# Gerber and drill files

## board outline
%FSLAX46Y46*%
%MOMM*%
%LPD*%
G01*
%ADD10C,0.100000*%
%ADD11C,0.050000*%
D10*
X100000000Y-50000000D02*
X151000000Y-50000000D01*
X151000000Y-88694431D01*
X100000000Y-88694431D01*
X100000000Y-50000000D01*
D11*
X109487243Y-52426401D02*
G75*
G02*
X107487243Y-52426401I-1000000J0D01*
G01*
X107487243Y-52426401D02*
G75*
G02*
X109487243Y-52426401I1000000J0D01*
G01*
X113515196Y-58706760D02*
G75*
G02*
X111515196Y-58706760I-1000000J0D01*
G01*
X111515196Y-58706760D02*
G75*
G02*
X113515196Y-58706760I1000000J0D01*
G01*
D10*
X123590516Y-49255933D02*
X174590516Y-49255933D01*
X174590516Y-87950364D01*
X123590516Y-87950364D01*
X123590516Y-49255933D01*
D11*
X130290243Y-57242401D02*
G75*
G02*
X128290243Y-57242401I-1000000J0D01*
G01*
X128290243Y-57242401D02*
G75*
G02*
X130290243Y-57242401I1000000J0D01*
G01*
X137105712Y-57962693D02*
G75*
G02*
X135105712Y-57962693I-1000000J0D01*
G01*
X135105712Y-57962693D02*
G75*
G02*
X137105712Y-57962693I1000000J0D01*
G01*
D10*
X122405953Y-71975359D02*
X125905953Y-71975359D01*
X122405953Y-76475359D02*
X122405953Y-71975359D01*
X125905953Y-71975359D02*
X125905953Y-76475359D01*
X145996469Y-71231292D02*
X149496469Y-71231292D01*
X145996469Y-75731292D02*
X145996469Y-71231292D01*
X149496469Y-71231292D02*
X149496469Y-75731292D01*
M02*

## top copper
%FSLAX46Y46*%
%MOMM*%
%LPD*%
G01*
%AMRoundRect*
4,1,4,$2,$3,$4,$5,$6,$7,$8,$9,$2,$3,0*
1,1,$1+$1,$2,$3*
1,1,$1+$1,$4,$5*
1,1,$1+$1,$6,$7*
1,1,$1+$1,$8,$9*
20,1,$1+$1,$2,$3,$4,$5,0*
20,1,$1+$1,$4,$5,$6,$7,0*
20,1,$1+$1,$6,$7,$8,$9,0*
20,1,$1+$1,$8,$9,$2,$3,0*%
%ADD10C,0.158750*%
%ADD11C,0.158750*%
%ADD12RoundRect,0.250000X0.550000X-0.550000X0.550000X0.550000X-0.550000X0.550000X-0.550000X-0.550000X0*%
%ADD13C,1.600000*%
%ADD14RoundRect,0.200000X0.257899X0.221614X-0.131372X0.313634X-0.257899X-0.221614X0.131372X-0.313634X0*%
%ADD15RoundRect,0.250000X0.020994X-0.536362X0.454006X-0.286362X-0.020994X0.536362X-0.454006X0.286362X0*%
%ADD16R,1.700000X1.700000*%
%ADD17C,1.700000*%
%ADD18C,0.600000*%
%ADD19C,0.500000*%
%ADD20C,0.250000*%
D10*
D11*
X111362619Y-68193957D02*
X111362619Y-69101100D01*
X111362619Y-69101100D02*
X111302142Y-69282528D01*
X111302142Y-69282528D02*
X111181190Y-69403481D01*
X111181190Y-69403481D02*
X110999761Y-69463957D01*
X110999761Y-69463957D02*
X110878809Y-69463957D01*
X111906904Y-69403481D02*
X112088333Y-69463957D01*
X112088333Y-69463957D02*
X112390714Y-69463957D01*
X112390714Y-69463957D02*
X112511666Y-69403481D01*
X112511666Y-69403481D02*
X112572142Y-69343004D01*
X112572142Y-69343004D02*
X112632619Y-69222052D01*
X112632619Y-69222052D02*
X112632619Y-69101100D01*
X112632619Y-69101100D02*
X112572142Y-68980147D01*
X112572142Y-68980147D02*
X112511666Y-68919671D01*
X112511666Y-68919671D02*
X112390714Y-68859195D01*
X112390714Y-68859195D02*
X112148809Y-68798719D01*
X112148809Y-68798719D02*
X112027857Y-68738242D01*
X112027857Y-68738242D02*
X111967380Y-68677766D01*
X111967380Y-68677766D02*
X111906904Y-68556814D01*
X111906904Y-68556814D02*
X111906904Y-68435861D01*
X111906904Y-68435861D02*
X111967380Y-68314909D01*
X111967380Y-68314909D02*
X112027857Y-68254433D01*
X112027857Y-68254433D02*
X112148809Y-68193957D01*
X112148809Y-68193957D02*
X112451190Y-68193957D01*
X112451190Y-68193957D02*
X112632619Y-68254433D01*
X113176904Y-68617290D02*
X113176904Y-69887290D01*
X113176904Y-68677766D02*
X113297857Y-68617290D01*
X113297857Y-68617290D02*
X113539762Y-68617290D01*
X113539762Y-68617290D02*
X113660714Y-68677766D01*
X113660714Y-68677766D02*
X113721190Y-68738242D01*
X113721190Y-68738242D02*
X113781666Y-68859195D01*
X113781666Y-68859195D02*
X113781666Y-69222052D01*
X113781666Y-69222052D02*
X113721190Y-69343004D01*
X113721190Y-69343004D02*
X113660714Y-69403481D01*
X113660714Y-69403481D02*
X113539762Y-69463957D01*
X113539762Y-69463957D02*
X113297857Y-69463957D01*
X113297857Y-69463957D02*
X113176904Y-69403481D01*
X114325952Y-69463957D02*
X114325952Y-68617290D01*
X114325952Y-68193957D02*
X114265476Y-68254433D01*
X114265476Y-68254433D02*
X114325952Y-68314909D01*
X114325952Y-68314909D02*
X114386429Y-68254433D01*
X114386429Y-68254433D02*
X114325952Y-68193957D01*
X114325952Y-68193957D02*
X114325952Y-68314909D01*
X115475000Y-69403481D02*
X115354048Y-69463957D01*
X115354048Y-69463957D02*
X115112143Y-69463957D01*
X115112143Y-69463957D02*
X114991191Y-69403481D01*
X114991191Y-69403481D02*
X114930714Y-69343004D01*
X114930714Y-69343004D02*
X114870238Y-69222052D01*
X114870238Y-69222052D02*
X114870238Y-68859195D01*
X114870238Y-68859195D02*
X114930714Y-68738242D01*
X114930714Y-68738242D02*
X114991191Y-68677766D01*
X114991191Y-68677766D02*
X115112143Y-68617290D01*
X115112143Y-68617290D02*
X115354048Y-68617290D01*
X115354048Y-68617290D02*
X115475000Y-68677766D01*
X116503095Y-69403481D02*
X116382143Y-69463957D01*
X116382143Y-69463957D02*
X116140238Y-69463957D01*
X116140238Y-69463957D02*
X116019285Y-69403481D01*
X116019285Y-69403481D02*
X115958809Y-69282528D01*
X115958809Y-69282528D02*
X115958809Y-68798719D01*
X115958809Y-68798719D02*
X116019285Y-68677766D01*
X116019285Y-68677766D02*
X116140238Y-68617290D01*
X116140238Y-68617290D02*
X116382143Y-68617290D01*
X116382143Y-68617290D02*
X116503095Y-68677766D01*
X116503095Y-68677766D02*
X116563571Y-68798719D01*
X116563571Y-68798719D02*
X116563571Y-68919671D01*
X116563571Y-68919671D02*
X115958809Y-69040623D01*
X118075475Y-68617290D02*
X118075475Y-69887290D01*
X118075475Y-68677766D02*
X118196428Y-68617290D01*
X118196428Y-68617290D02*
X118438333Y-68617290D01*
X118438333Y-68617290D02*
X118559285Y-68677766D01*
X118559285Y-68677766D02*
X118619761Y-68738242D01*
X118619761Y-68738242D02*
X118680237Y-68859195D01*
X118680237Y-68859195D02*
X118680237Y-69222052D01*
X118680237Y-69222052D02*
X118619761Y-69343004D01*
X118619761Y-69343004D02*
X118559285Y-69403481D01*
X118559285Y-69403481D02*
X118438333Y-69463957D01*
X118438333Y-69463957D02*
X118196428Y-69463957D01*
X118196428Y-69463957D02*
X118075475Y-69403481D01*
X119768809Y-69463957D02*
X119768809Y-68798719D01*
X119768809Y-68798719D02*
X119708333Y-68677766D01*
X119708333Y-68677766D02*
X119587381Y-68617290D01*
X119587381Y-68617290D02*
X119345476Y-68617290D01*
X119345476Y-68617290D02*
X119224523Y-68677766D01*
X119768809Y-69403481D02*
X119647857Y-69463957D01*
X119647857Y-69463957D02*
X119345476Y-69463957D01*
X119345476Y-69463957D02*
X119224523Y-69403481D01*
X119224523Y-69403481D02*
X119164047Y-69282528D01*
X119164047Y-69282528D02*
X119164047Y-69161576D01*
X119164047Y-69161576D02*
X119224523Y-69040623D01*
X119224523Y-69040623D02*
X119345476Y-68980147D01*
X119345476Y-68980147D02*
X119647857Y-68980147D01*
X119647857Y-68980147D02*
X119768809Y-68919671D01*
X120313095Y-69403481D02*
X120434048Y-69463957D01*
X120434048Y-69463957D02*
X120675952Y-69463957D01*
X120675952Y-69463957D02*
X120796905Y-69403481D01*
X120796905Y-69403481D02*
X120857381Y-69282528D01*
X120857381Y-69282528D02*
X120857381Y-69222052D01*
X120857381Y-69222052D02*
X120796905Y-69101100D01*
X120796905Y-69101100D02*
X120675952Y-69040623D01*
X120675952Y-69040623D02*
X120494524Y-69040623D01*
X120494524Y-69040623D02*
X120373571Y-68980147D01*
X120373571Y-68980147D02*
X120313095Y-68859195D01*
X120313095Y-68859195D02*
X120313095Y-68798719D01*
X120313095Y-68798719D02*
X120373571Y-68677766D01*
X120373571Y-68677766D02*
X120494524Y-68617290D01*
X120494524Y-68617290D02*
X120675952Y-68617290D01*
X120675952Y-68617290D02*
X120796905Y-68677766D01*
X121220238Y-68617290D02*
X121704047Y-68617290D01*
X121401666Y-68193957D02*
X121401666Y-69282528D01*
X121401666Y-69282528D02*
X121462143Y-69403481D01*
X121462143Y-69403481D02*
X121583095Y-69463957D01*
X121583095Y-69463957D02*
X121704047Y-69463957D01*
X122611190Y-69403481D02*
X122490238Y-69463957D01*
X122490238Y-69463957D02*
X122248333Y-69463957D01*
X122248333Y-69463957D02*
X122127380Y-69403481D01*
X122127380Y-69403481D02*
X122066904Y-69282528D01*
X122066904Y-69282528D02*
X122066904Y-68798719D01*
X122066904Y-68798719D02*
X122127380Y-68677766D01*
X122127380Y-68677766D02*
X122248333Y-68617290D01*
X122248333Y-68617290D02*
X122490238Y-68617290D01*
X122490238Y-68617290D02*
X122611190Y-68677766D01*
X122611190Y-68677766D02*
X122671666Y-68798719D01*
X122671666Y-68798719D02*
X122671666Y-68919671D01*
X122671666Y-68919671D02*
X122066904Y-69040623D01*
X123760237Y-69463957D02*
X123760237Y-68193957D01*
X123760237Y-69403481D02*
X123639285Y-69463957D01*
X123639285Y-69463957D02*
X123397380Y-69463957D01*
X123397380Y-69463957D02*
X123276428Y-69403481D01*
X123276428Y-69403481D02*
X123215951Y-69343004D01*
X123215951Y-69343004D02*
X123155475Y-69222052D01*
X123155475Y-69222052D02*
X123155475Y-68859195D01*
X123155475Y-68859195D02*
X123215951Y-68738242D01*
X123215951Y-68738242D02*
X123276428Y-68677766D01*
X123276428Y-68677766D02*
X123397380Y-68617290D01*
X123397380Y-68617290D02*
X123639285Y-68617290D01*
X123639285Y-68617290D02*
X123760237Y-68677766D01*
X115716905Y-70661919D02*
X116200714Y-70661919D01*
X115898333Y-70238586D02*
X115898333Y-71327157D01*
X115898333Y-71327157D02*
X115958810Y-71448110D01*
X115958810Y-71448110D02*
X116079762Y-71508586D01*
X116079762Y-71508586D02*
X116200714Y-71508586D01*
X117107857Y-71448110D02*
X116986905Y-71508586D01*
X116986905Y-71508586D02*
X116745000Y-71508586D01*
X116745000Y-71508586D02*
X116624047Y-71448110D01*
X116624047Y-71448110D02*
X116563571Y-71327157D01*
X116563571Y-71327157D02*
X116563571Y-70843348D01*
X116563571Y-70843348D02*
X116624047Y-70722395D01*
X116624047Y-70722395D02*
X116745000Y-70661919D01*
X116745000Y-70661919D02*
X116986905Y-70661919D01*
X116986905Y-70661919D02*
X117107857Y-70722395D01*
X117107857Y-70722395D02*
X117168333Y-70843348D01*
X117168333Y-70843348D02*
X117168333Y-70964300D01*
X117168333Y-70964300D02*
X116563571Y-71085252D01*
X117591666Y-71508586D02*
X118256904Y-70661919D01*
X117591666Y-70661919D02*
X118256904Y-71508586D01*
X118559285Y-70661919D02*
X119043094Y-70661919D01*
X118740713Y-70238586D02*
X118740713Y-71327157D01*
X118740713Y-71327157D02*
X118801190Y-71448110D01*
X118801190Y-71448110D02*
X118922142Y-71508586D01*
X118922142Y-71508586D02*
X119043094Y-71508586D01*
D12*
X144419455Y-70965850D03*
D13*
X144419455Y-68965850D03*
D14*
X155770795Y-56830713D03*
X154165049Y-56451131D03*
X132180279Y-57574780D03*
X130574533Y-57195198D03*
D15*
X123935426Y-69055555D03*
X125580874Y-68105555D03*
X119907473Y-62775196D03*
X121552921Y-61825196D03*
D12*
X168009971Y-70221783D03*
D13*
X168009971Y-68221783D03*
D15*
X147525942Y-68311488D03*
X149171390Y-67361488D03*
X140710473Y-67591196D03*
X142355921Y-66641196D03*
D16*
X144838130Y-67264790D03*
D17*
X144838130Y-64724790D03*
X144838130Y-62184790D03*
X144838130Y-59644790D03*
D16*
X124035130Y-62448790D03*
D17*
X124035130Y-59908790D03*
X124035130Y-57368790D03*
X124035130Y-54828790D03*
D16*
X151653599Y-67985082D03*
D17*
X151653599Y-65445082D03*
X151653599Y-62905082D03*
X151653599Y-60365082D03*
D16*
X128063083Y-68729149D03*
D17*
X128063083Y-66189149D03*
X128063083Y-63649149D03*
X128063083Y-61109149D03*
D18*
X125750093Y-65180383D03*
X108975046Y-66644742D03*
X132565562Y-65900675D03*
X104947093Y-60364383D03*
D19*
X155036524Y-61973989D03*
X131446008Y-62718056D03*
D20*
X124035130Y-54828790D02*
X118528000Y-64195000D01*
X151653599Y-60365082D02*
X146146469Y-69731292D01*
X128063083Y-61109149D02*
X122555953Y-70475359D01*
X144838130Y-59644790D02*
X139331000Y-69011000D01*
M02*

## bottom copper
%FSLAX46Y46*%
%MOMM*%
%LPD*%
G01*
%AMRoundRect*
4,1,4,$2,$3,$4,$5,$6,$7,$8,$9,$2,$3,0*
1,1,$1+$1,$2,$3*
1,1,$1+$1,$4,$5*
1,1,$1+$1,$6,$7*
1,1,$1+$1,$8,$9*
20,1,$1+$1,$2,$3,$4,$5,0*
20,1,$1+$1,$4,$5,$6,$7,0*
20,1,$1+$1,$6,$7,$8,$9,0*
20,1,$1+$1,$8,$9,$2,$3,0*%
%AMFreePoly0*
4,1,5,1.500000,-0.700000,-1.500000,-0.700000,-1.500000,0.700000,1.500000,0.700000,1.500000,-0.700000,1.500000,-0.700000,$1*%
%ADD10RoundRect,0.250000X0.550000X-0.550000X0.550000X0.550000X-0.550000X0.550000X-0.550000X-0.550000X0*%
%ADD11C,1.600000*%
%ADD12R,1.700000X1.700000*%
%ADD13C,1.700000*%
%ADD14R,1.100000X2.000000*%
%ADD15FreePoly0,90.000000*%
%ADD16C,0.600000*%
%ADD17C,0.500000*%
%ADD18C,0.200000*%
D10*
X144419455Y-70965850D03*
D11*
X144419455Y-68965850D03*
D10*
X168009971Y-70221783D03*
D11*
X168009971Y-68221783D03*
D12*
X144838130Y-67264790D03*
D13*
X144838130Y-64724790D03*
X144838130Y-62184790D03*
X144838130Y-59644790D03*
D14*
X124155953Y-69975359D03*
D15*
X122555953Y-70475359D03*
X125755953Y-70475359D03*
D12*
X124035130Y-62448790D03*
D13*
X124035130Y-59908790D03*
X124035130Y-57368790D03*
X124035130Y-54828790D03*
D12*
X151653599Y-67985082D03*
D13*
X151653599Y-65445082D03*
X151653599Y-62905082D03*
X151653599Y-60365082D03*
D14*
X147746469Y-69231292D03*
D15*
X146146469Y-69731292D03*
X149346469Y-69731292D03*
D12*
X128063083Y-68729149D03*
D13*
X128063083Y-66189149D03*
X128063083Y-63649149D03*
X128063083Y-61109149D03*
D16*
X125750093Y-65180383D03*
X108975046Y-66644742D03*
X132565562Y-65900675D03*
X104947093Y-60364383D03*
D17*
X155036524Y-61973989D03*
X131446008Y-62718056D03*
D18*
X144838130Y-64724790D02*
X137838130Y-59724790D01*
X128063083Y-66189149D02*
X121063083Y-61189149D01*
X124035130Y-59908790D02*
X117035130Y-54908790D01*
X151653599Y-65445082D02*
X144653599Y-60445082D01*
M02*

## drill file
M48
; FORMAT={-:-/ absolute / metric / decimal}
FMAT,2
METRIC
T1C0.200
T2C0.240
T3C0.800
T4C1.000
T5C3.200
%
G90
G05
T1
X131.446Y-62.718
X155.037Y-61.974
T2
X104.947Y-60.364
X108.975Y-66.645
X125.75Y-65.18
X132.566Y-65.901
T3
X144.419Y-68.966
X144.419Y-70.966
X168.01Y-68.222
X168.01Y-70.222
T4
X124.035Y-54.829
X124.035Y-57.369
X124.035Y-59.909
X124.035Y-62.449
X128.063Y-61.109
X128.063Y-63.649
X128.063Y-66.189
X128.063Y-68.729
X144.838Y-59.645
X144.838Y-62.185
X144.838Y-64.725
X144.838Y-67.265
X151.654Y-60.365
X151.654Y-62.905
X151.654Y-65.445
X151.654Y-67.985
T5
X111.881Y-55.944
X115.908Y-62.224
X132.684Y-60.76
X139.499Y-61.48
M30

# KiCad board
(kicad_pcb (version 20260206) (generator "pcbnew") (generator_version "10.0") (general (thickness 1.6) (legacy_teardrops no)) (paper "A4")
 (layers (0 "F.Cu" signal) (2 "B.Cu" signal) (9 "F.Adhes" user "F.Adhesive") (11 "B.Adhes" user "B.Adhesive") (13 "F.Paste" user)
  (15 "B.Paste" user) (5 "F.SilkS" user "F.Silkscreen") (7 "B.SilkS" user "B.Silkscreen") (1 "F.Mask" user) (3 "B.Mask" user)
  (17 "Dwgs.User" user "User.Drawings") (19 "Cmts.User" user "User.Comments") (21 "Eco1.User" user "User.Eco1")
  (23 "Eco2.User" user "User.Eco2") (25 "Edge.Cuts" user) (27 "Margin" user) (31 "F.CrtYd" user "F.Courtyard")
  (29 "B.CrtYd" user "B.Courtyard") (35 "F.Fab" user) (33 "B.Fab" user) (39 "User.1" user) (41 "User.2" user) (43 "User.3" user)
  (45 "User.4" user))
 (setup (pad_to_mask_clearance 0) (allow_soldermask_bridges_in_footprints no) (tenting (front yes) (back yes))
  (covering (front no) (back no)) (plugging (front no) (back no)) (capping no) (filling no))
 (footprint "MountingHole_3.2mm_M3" (layer "F.Cu") (at 132.683531 60.759708 45)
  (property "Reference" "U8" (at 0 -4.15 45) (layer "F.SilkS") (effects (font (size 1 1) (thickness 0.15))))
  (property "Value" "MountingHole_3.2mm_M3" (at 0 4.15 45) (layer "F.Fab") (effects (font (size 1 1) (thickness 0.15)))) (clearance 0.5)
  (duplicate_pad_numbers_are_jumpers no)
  (pad "" np_thru_hole circle (at 0 0 45) (size 3.2 3.2) (drill 3.2) (layers "*.Cu" "*.Mask")))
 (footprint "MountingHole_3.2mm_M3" (layer "F.Cu") (at 139.499 61.48 45)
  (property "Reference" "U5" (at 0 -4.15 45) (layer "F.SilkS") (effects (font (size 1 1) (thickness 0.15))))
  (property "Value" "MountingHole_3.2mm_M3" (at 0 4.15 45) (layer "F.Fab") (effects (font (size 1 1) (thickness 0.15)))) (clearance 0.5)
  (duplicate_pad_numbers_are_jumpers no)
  (pad "" np_thru_hole circle (at 0 0 45) (size 3.2 3.2) (drill 3.2) (layers "*.Cu" "*.Mask")))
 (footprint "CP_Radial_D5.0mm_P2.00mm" (layer "F.Cu") (at 144.419455 70.96585 90)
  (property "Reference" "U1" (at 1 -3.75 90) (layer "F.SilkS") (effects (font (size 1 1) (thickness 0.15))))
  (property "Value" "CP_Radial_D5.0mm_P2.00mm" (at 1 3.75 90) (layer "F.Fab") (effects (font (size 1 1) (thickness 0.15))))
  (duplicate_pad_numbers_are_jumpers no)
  (pad "1" thru_hole roundrect (at 0 0 90) (size 1.6 1.6) (drill 0.8) (layers "*.Cu" "*.Mask") (remove_unused_layers no)
   (roundrect_rratio 0.15625) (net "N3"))
  (pad "2" thru_hole circle (at 2 0 90) (size 1.6 1.6) (drill 0.8) (layers "*.Cu" "*.Mask") (remove_unused_layers no) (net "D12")))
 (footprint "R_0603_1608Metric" (layer "F.Cu") (at 154.967922 56.640922 166.7)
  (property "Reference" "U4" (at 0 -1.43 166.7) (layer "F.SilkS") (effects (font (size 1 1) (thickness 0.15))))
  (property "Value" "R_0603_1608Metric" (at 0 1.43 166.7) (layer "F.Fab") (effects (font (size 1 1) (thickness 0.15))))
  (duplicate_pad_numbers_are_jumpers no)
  (pad "1" smd roundrect (at -0.825 0 166.7) (size 0.8 0.95) (layers "F.Cu" "F.Mask" "F.Paste") (roundrect_rratio 0.25) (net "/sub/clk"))
  (pad "2" smd roundrect (at 0.825 0 166.7) (size 0.8 0.95) (layers "F.Cu" "F.Mask" "F.Paste") (roundrect_rratio 0.25) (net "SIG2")))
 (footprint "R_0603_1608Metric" (layer "F.Cu") (at 131.377406 57.384989 166.7)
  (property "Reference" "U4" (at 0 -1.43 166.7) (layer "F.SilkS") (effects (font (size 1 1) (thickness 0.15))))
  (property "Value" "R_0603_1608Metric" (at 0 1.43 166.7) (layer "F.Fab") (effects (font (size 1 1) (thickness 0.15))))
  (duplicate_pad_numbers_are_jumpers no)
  (pad "1" smd roundrect (at -0.825 0 166.7) (size 0.8 0.95) (layers "F.Cu" "F.Mask" "F.Paste") (roundrect_rratio 0.25) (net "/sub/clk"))
  (pad "2" smd roundrect (at 0.825 0 166.7) (size 0.8 0.95) (layers "F.Cu" "F.Mask" "F.Paste") (roundrect_rratio 0.25) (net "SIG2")))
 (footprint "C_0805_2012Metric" (layer "F.Cu") (at 124.75815 68.580555 30)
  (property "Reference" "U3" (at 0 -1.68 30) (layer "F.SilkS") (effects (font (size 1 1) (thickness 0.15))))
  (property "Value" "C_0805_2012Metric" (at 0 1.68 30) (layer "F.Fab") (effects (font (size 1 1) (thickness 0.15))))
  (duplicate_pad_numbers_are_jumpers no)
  (pad "1" smd roundrect (at -0.95 0 30) (size 1 1.45) (layers "F.Cu" "F.Mask" "F.Paste") (roundrect_rratio 0.25) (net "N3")
   (clearance 0.35))
  (pad "2" smd roundrect (at 0.95 0 30) (size 1 1.45) (layers "F.Cu" "F.Mask" "F.Paste") (roundrect_rratio 0.25)))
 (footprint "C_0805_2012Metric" (layer "F.Cu") (at 120.730197 62.300196 30)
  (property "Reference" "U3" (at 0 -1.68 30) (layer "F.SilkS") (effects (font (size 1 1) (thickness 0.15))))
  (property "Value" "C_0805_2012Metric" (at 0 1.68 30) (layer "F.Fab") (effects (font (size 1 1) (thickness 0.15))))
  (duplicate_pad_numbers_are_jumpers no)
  (pad "1" smd roundrect (at -0.95 0 30) (size 1 1.45) (layers "F.Cu" "F.Mask" "F.Paste") (roundrect_rratio 0.25) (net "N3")
   (clearance 0.35))
  (pad "2" smd roundrect (at 0.95 0 30) (size 1 1.45) (layers "F.Cu" "F.Mask" "F.Paste") (roundrect_rratio 0.25)))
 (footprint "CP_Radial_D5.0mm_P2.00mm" (layer "F.Cu") (at 168.009971 70.221783 90)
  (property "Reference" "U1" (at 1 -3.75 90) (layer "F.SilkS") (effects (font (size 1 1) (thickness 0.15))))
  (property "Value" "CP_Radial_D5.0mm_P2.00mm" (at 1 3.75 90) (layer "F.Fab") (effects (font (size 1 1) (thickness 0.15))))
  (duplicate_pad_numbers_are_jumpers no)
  (pad "1" thru_hole roundrect (at 0 0 90) (size 1.6 1.6) (drill 0.8) (layers "*.Cu" "*.Mask") (remove_unused_layers no)
   (roundrect_rratio 0.15625) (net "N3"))
  (pad "2" thru_hole circle (at 2 0 90) (size 1.6 1.6) (drill 0.8) (layers "*.Cu" "*.Mask") (remove_unused_layers no) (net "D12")))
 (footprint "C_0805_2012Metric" (layer "F.Cu") (at 148.348666 67.836488 30)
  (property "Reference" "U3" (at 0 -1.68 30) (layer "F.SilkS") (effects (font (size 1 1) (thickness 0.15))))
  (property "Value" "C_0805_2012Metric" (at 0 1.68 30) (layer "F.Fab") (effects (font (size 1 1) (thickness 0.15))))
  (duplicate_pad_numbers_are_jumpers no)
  (pad "1" smd roundrect (at -0.95 0 30) (size 1 1.45) (layers "F.Cu" "F.Mask" "F.Paste") (roundrect_rratio 0.25) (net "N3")
   (clearance 0.35))
  (pad "2" smd roundrect (at 0.95 0 30) (size 1 1.45) (layers "F.Cu" "F.Mask" "F.Paste") (roundrect_rratio 0.25)))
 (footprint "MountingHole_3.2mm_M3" (layer "F.Cu") (at 115.908484 62.224067 45)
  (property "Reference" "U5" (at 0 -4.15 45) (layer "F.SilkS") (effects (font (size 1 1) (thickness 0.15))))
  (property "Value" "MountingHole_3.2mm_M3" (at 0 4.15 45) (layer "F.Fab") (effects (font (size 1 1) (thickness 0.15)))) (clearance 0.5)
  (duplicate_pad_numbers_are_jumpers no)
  (pad "" np_thru_hole circle (at 0 0 45) (size 3.2 3.2) (drill 3.2) (layers "*.Cu" "*.Mask")))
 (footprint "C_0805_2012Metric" (layer "F.Cu") (at 141.533197 67.116196 30)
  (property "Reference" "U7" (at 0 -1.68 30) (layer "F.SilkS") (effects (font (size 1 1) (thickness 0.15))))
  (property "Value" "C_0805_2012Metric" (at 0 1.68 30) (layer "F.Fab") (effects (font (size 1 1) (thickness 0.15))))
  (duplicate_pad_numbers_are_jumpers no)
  (pad "1" smd roundrect (at -0.95 0 30) (size 1 1.45) (layers "F.Cu" "F.Mask" "F.Paste") (roundrect_rratio 0.25) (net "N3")
   (clearance 0.35))
  (pad "2" smd roundrect (at 0.95 0 30) (size 1 1.45) (layers "F.Cu" "F.Mask" "F.Paste") (roundrect_rratio 0.25)))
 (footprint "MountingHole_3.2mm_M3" (layer "F.Cu") (at 111.880531 55.943708 45)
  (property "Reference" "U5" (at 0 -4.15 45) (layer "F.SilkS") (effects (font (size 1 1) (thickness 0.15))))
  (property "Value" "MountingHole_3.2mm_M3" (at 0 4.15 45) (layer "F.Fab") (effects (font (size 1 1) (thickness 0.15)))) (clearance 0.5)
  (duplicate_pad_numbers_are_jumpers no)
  (pad "" np_thru_hole circle (at 0 0 45) (size 3.2 3.2) (drill 3.2) (layers "*.Cu" "*.Mask")))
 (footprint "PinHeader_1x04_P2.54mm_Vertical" (layer "B.Cu") (at 144.83813 67.26479)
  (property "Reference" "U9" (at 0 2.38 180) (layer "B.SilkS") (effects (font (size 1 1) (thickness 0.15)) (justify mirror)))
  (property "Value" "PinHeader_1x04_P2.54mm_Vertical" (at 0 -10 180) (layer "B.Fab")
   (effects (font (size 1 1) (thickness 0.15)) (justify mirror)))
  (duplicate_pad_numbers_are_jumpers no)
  (pad "1" thru_hole rect (at 0 0) (size 1.7 1.7) (drill 1) (layers "*.Cu" "*.Mask") (remove_unused_layers no) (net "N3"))
  (pad "2" thru_hole circle (at 0 -2.54) (size 1.7 1.7) (drill 1) (layers "*.Cu" "*.Mask") (remove_unused_layers no) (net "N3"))
  (pad "3" thru_hole circle (at 0 -5.08) (size 1.7 1.7) (drill 1) (layers "*.Cu" "*.Mask") (remove_unused_layers no) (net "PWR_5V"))
  (pad "4" thru_hole circle (at 0 -7.62) (size 1.7 1.7) (drill 1) (layers "*.Cu" "*.Mask") (remove_unused_layers no)))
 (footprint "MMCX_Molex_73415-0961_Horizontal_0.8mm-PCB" (layer "B.Cu") (at 124.155953 72.725359 90)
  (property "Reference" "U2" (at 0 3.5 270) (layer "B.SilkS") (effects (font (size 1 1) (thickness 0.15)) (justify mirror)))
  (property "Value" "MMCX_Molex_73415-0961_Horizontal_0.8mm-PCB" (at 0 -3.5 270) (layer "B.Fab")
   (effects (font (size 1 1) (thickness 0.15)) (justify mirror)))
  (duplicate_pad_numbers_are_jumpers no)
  (fp_line (start 0.75 -1.75) (end 0.75 1.75) (stroke (width 0.1) (type solid)) (layer "Edge.Cuts"))
  (fp_line (start -3.75 -1.75) (end 0.75 -1.75) (stroke (width 0.1) (type solid)) (layer "Edge.Cuts"))
  (fp_line (start 0.75 1.75) (end -3.75 1.75) (stroke (width 0.1) (type solid)) (layer "Edge.Cuts"))
  (pad "1" smd rect (at 2.75 0 90) (size 2 1.1) (layers "B.Cu" "B.Mask" "B.Paste") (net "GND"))
  (pad "2" smd custom (at 2.25 -1.6 90) (size 3 1.4) (layers "B.Cu" "B.Mask" "B.Paste") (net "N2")
   (options (clearance outline) (anchor rect)) (primitives))
  (pad "2" smd custom (at 2.25 1.6 90) (size 3 1.4) (layers "B.Cu" "B.Mask" "B.Paste") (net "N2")
   (options (clearance outline) (anchor rect)) (primitives)))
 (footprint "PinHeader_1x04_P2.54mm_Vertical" (layer "B.Cu") (at 124.03513 62.44879)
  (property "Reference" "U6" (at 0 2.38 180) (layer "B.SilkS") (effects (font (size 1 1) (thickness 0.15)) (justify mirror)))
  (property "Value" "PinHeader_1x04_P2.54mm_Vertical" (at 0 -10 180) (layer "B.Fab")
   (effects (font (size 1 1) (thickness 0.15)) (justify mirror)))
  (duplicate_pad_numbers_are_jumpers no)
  (pad "1" thru_hole rect (at 0 0) (size 1.7 1.7) (drill 1) (layers "*.Cu" "*.Mask") (remove_unused_layers no) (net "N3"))
  (pad "2" thru_hole circle (at 0 -2.54) (size 1.7 1.7) (drill 1) (layers "*.Cu" "*.Mask") (remove_unused_layers no) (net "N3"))
  (pad "3" thru_hole circle (at 0 -5.08) (size 1.7 1.7) (drill 1) (layers "*.Cu" "*.Mask") (remove_unused_layers no) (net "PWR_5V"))
  (pad "4" thru_hole circle (at 0 -7.62) (size 1.7 1.7) (drill 1) (layers "*.Cu" "*.Mask") (remove_unused_layers no)))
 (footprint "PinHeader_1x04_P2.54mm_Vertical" (layer "B.Cu") (at 151.653599 67.985082)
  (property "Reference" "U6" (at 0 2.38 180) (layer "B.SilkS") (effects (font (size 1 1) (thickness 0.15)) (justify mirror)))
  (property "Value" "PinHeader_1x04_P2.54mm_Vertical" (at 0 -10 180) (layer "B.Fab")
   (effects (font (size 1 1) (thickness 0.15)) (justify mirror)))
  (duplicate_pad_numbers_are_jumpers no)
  (pad "1" thru_hole rect (at 0 0) (size 1.7 1.7) (drill 1) (layers "*.Cu" "*.Mask") (remove_unused_layers no) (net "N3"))
  (pad "2" thru_hole circle (at 0 -2.54) (size 1.7 1.7) (drill 1) (layers "*.Cu" "*.Mask") (remove_unused_layers no) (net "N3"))
  (pad "3" thru_hole circle (at 0 -5.08) (size 1.7 1.7) (drill 1) (layers "*.Cu" "*.Mask") (remove_unused_layers no) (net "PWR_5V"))
  (pad "4" thru_hole circle (at 0 -7.62) (size 1.7 1.7) (drill 1) (layers "*.Cu" "*.Mask") (remove_unused_layers no)))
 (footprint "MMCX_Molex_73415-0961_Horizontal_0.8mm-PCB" (layer "B.Cu") (at 147.746469 71.981292 90)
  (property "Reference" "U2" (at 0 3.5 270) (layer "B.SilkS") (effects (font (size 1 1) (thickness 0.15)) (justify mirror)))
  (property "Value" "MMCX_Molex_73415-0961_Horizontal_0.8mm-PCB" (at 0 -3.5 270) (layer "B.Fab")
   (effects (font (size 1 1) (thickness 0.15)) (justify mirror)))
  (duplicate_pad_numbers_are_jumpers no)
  (fp_line (start 0.75 -1.75) (end 0.75 1.75) (stroke (width 0.1) (type solid)) (layer "Edge.Cuts"))
  (fp_line (start -3.75 -1.75) (end 0.75 -1.75) (stroke (width 0.1) (type solid)) (layer "Edge.Cuts"))
  (fp_line (start 0.75 1.75) (end -3.75 1.75) (stroke (width 0.1) (type solid)) (layer "Edge.Cuts"))
  (pad "1" smd rect (at 2.75 0 90) (size 2 1.1) (layers "B.Cu" "B.Mask" "B.Paste") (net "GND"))
  (pad "2" smd custom (at 2.25 -1.6 90) (size 3 1.4) (layers "B.Cu" "B.Mask" "B.Paste") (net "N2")
   (options (clearance outline) (anchor rect)) (primitives))
  (pad "2" smd custom (at 2.25 1.6 90) (size 3 1.4) (layers "B.Cu" "B.Mask" "B.Paste") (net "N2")
   (options (clearance outline) (anchor rect)) (primitives)))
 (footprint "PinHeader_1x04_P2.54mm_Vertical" (layer "B.Cu") (at 128.063083 68.729149)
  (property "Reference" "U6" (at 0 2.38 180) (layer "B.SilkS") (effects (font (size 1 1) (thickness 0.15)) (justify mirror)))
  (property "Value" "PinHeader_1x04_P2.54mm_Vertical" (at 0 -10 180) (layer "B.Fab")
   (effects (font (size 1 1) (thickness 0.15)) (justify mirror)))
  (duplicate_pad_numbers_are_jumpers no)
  (pad "1" thru_hole rect (at 0 0) (size 1.7 1.7) (drill 1) (layers "*.Cu" "*.Mask") (remove_unused_layers no) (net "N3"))
  (pad "2" thru_hole circle (at 0 -2.54) (size 1.7 1.7) (drill 1) (layers "*.Cu" "*.Mask") (remove_unused_layers no) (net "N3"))
  (pad "3" thru_hole circle (at 0 -5.08) (size 1.7 1.7) (drill 1) (layers "*.Cu" "*.Mask") (remove_unused_layers no) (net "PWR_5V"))
  (pad "4" thru_hole circle (at 0 -7.62) (size 1.7 1.7) (drill 1) (layers "*.Cu" "*.Mask") (remove_unused_layers no)))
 (gr_rect (start 100 50) (end 151 88.694431) (stroke (width 0.1) (type default)) (fill no) (layer "Edge.Cuts"))
 (gr_circle (center 108.487243 52.426401) (end 109.487243 52.426401) (stroke (width 0.05) (type default)) (fill no) (layer "Edge.Cuts"))
 (gr_circle (center 112.515196 58.70676) (end 113.515196 58.70676) (stroke (width 0.05) (type default)) (fill no) (layer "Edge.Cuts"))
 (gr_rect (start 123.590516 49.255933) (end 174.590516 87.950364) (stroke (width 0.1) (type default)) (fill no) (layer "Edge.Cuts"))
 (gr_circle (center 129.290243 57.242401) (end 130.290243 57.242401) (stroke (width 0.05) (type default)) (fill no) (layer "Edge.Cuts"))
 (gr_circle (center 136.105712 57.962693) (end 137.105712 57.962693) (stroke (width 0.05) (type default)) (fill no) (layer "Edge.Cuts"))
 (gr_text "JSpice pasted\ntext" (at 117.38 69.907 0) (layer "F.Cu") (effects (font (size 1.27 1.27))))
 (segment (start 124.03513 54.82879) (end 118.528 64.195) (width 0.25) (layer "F.Cu") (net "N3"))
 (segment (start 151.653599 60.365082) (end 146.146469 69.731292) (width 0.25) (layer "F.Cu") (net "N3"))
 (segment (start 128.063083 61.109149) (end 122.555953 70.475359) (width 0.25) (layer "F.Cu") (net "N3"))
 (segment (start 144.83813 59.64479) (end 139.331 69.011) (width 0.25) (layer "F.Cu") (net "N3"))
 (via (at 125.750093 65.180383) (size 0.6) (drill 0.24) (layers "F.Cu" "B.Cu") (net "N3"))
 (segment (start 144.83813 64.72479) (end 137.83813 59.72479) (width 0.2) (layer "B.Cu") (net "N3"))
 (segment (start 128.063083 66.189149) (end 121.063083 61.189149) (width 0.2) (layer "B.Cu") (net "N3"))
 (segment (start 124.03513 59.90879) (end 117.03513 54.90879) (width 0.2) (layer "B.Cu") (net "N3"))
 (segment (start 151.653599 65.445082) (end 144.653599 60.445082) (width 0.2) (layer "B.Cu") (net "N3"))
 (via (at 108.975046 66.644742) (size 0.6) (drill 0.24) (layers "F.Cu" "B.Cu") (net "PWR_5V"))
 (via (at 132.565562 65.900675) (size 0.6) (drill 0.24) (layers "F.Cu" "B.Cu") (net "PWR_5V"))
 (via (at 104.947093 60.364383) (size 0.6) (drill 0.24) (layers "F.Cu" "B.Cu") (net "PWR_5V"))
 (via (at 155.036524 61.973989) (size 0.5) (drill 0.2) (layers "F.Cu" "B.Cu") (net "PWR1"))
 (via (at 131.446008 62.718056) (size 0.5) (drill 0.2) (layers "F.Cu" "B.Cu") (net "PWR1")))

